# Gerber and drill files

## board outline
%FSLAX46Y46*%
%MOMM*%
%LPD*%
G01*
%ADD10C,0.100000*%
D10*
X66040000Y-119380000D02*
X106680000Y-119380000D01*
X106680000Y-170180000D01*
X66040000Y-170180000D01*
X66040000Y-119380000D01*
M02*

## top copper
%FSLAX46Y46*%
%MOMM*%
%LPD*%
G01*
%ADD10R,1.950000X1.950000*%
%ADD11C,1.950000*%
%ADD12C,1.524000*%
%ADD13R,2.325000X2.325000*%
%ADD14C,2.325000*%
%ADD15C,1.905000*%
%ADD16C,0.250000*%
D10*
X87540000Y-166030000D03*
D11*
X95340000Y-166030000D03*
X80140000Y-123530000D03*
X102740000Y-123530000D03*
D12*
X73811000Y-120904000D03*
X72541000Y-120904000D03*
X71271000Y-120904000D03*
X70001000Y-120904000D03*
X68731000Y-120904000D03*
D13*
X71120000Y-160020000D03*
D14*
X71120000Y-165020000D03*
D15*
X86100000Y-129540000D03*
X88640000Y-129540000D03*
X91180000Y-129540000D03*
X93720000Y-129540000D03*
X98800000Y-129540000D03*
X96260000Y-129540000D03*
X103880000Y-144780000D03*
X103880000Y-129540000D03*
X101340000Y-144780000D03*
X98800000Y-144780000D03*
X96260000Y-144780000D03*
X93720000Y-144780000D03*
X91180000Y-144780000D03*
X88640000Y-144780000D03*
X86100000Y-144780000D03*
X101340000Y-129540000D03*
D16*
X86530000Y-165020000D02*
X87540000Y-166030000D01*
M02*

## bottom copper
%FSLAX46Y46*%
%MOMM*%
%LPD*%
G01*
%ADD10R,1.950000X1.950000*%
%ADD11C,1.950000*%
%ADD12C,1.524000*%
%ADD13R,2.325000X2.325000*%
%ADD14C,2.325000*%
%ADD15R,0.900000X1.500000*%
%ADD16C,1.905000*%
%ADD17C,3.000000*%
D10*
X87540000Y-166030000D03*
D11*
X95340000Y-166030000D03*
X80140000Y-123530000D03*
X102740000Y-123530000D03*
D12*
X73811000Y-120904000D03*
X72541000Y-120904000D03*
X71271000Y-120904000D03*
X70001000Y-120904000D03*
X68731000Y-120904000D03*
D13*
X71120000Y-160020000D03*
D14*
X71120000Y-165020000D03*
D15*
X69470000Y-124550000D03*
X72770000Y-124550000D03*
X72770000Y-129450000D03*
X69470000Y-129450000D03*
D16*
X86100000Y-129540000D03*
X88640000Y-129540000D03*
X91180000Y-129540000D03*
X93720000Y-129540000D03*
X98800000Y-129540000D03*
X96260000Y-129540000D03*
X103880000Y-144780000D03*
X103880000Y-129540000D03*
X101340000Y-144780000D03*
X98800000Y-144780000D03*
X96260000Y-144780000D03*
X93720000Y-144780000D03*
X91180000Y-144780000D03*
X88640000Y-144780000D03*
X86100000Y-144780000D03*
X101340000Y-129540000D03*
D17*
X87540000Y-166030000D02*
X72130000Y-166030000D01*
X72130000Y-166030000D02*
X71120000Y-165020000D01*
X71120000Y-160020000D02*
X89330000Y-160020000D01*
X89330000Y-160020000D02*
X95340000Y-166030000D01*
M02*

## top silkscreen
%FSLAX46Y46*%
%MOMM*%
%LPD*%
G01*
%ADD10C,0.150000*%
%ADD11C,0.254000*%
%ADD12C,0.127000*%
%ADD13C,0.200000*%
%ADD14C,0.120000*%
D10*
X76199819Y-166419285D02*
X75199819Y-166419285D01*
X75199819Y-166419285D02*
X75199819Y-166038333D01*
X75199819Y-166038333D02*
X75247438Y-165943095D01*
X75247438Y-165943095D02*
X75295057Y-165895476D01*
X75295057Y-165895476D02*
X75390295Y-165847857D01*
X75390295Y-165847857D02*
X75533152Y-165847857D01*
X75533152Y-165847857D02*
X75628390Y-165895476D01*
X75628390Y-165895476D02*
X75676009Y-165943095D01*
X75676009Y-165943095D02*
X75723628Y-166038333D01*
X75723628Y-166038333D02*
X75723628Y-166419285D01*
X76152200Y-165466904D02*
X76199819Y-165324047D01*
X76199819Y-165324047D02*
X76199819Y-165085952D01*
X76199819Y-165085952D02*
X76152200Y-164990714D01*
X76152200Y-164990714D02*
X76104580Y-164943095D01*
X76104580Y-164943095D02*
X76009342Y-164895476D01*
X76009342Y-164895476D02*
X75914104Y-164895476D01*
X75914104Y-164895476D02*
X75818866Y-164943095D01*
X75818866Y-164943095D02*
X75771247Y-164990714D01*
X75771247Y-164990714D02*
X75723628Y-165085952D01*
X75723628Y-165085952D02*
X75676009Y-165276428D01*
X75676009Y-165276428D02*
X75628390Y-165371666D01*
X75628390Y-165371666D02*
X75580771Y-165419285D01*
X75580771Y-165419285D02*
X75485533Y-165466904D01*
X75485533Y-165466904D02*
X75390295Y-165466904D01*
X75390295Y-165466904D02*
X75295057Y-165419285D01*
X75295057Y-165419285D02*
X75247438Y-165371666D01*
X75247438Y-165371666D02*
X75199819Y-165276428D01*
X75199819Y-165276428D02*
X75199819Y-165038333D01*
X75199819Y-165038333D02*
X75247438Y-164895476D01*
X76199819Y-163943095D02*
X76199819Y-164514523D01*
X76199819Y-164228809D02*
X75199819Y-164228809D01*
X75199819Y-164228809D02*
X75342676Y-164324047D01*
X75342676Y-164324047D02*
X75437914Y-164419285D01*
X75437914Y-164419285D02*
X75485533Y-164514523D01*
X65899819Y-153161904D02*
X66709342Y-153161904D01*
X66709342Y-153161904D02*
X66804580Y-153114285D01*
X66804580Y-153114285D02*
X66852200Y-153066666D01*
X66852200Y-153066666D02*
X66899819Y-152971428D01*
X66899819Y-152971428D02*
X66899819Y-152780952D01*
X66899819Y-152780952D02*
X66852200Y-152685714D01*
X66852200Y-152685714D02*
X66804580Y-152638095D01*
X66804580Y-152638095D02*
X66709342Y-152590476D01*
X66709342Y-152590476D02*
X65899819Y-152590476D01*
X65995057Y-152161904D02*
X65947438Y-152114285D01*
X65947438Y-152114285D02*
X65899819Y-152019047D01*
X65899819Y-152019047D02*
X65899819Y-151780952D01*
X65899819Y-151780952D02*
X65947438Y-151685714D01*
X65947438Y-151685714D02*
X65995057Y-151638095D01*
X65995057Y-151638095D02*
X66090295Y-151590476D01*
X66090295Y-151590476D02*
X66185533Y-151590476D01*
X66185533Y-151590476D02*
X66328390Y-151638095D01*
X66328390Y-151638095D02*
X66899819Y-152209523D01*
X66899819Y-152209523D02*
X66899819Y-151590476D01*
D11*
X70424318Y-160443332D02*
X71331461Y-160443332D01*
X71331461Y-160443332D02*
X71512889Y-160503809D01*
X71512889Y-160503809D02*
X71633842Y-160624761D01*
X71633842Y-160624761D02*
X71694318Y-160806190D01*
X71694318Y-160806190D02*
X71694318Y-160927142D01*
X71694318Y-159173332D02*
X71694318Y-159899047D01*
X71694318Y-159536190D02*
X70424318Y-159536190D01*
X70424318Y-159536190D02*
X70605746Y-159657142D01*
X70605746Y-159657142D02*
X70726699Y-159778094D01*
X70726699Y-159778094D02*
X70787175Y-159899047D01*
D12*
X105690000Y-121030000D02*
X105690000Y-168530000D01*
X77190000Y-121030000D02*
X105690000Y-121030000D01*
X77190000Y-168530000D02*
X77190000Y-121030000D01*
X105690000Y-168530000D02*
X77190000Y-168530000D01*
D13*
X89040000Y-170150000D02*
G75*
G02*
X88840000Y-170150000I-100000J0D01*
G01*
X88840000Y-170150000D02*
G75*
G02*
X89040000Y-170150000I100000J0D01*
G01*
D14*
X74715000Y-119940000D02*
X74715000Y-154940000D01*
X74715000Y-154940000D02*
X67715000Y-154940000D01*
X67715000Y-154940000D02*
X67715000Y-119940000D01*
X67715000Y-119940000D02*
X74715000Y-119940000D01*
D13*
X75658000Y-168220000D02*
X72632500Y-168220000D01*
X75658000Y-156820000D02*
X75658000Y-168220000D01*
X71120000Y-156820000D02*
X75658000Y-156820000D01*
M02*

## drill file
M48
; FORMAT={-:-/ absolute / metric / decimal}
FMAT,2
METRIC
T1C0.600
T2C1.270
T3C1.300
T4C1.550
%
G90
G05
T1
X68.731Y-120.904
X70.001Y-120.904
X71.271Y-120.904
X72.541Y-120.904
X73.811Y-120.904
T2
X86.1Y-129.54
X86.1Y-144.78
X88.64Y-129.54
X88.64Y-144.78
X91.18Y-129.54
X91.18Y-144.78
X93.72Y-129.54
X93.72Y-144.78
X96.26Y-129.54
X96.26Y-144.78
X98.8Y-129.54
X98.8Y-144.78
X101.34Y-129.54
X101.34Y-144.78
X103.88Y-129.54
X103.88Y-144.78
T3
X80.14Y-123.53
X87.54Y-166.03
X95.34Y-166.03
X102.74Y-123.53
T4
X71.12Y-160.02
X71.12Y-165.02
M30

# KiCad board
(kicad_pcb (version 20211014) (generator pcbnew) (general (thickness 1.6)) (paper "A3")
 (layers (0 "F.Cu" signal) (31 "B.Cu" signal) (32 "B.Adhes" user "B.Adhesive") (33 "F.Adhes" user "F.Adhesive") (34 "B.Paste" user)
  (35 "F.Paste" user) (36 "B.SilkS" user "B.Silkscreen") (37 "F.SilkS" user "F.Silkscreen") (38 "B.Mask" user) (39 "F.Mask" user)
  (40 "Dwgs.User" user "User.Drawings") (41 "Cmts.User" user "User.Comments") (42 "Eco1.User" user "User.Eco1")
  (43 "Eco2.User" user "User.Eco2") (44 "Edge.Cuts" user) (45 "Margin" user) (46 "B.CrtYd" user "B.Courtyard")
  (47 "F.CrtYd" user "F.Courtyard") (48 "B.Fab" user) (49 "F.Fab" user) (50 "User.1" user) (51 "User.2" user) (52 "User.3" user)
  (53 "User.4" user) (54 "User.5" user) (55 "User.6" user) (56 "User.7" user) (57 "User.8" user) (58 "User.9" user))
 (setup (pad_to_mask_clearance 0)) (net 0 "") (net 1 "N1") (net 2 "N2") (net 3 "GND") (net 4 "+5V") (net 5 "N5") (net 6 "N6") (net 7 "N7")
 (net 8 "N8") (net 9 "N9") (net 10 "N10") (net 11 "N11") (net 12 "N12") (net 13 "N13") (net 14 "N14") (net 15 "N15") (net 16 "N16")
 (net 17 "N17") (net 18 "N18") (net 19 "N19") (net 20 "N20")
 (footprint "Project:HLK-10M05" (layer "F.Cu") (at 91.44 144.78 90)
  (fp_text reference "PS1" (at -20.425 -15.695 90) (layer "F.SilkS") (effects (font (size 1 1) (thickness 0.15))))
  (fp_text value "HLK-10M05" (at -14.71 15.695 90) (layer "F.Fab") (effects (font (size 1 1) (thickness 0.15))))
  (fp_line (start 23.75 14.25) (end -23.75 14.25) (layer "F.SilkS") (width 0.127))
  (fp_line (start 23.75 -14.25) (end 23.75 14.25) (layer "F.SilkS") (width 0.127))
  (fp_line (start -23.75 -14.25) (end 23.75 -14.25) (layer "F.SilkS") (width 0.127))
  (fp_line (start -23.75 14.25) (end -23.75 -14.25) (layer "F.SilkS") (width 0.127))
  (fp_circle (center -25.37 -2.5) (end -25.27 -2.5) (layer "F.SilkS") (width 0.2) (fill none))
  (pad "1" thru_hole rect (at -21.25 -3.9 90) (size 1.95 1.95) (drill 1.3) (layers *.Cu *.Mask) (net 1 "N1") (solder_mask_margin 0.102))
  (pad "2" thru_hole circle (at -21.25 3.9 90) (size 1.95 1.95) (drill 1.3) (layers *.Cu *.Mask) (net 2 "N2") (solder_mask_margin 0.102))
  (pad "3" thru_hole circle (at 21.25 -11.3 90) (size 1.95 1.95) (drill 1.3) (layers *.Cu *.Mask) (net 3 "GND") (solder_mask_margin 0.102))
  (pad "4" thru_hole circle (at 21.25 11.3 90) (size 1.95 1.95) (drill 1.3) (layers *.Cu *.Mask) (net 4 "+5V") (solder_mask_margin 0.102)))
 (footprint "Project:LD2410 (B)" (layer "F.Cu") (at 67.715 154.94 90)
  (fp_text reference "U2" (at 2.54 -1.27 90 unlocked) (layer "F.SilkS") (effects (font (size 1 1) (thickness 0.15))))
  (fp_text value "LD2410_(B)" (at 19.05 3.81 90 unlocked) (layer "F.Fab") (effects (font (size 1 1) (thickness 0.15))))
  (fp_line (start 35 7) (end 0 7) (layer "F.SilkS") (width 0.12))
  (fp_line (start 0 7) (end 0 0) (layer "F.SilkS") (width 0.12))
  (fp_line (start 0 0) (end 35 0) (layer "F.SilkS") (width 0.12))
  (fp_line (start 35 0) (end 35 7) (layer "F.SilkS") (width 0.12))
  (pad "1" thru_hole circle (at 34.036 6.096 90) (size 1.524 1.524) (drill 0.6) (layers *.Cu *.Mask) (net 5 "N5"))
  (pad "2" thru_hole circle (at 34.036 4.826 90) (size 1.524 1.524) (drill 0.6) (layers *.Cu *.Mask) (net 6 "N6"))
  (pad "3" thru_hole circle (at 34.036 3.556 90) (size 1.524 1.524) (drill 0.6) (layers *.Cu *.Mask) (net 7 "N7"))
  (pad "4" thru_hole circle (at 34.036 2.286 90) (size 1.524 1.524) (drill 0.6) (layers *.Cu *.Mask) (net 3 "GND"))
  (pad "5" thru_hole circle (at 34.036 1.016 90) (size 1.524 1.524) (drill oval 0.6) (layers *.Cu *.Mask) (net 4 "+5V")))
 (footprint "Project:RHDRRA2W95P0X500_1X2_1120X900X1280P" (layer "F.Cu") (at 71.12 160.02 -90)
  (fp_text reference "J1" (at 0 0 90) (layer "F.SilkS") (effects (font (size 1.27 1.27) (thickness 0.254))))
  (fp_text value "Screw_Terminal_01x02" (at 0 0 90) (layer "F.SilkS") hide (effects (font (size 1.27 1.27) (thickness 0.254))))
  (fp_line (start 8.2 -4.538) (end 8.2 -1.5125) (layer "F.SilkS") (width 0.2))
  (fp_line (start -3.2 -4.538) (end 8.2 -4.538) (layer "F.SilkS") (width 0.2))
  (fp_line (start -3.2 0) (end -3.2 -4.538) (layer "F.SilkS") (width 0.2))
  (pad "1" thru_hole rect locked (at 0 0 270) (size 2.325 2.325) (drill 1.55) (layers *.Cu *.Mask) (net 2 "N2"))
  (pad "2" thru_hole circle locked (at 5 0 270) (size 2.325 2.325) (drill 1.55) (layers *.Cu *.Mask) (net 1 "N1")))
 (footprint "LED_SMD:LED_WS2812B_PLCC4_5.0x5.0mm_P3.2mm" (layer "B.Cu") (at 71.12 127 -90)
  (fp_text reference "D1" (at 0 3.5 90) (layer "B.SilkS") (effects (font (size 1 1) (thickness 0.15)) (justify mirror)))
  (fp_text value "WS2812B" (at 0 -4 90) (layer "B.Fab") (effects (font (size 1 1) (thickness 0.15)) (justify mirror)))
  (pad "1" smd rect (at -2.45 1.65 270) (size 1.5 0.9) (layers "B.Cu" "B.Paste" "B.Mask") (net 3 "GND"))
  (pad "2" smd rect (at -2.45 -1.65 270) (size 1.5 0.9) (layers "B.Cu" "B.Paste" "B.Mask") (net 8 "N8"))
  (pad "3" smd rect (at 2.45 -1.65 270) (size 1.5 0.9) (layers "B.Cu" "B.Paste" "B.Mask") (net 4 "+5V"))
  (pad "4" smd rect (at 2.45 1.65 270) (size 1.5 0.9) (layers "B.Cu" "B.Paste" "B.Mask") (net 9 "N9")))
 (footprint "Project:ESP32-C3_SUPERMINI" (layer "B.Cu") (at 93.98 137.16 90)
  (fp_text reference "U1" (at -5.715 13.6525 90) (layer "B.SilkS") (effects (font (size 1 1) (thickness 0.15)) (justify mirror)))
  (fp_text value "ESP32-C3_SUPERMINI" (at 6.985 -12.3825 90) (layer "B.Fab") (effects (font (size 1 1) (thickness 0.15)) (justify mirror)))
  (pad "0" thru_hole circle (at 7.62 -7.88 90) (size 1.905 1.905) (drill 1.27) (layers *.Cu *.Mask) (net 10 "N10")
   (solder_mask_margin 0.102))
  (pad "1" thru_hole circle (at 7.62 -5.34 90) (size 1.905 1.905) (drill 1.27) (layers *.Cu *.Mask) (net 6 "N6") (solder_mask_margin 0.102))
  (pad "2" thru_hole circle (at 7.62 -2.8 90) (size 1.905 1.905) (drill 1.27) (layers *.Cu *.Mask) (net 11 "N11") (solder_mask_margin 0.102))
  (pad "3" thru_hole circle (at 7.62 -0.26 90) (size 1.905 1.905) (drill 1.27) (layers *.Cu *.Mask) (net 7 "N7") (solder_mask_margin 0.102))
  (pad "3.3" thru_hole circle (at 7.62 4.82 90) (size 1.905 1.905) (drill 1.27) (layers *.Cu *.Mask) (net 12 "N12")
   (solder_mask_margin 0.102))
  (pad "4" thru_hole circle (at 7.62 2.28 90) (size 1.905 1.905) (drill 1.27) (layers *.Cu *.Mask) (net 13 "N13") (solder_mask_margin 0.102))
  (pad "5" thru_hole circle (at -7.62 9.9 90) (size 1.905 1.905) (drill 1.27) (layers *.Cu *.Mask) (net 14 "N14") (solder_mask_margin 0.102))
  (pad "5V" thru_hole circle (at 7.62 9.9 90) (size 1.905 1.905) (drill 1.27) (layers *.Cu *.Mask) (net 4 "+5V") (solder_mask_margin 0.102))
  (pad "6" thru_hole circle (at -7.62 7.36 90) (size 1.905 1.905) (drill 1.27) (layers *.Cu *.Mask) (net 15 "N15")
   (solder_mask_margin 0.102))
  (pad "7" thru_hole circle (at -7.62 4.82 90) (size 1.905 1.905) (drill 1.27) (layers *.Cu *.Mask) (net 9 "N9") (solder_mask_margin 0.102))
  (pad "8" thru_hole circle (at -7.62 2.28 90) (size 1.905 1.905) (drill 1.27) (layers *.Cu *.Mask) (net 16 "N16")
   (solder_mask_margin 0.102))
  (pad "9" thru_hole circle (at -7.62 -0.26 90) (size 1.905 1.905) (drill 1.27) (layers *.Cu *.Mask) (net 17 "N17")
   (solder_mask_margin 0.102))
  (pad "10" thru_hole circle (at -7.62 -2.8 90) (size 1.905 1.905) (drill 1.27) (layers *.Cu *.Mask) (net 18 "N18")
   (solder_mask_margin 0.102))
  (pad "20" thru_hole circle (at -7.62 -5.34 90) (size 1.905 1.905) (drill 1.27) (layers *.Cu *.Mask) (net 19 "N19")
   (solder_mask_margin 0.102))
  (pad "21" thru_hole circle (at -7.62 -7.88 90) (size 1.905 1.905) (drill 1.27) (layers *.Cu *.Mask) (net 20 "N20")
   (solder_mask_margin 0.102))
  (pad "G" thru_hole circle (at 7.62 7.36 90) (size 1.905 1.905) (drill 1.27) (layers *.Cu *.Mask) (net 3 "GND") (solder_mask_margin 0.102)))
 (gr_rect (start 66.04 119.38) (end 106.68 170.18) (layer "Edge.Cuts") (width 0.1) (fill none))
 (segment (start 86.53 165.02) (end 87.54 166.03) (width 0.25) (layer "F.Cu") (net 1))
 (segment (start 87.54 166.03) (end 72.13 166.03) (width 3) (layer "B.Cu") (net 1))
 (segment (start 72.13 166.03) (end 71.12 165.02) (width 3) (layer "B.Cu") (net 1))
 (segment (start 71.12 160.02) (end 89.33 160.02) (width 3) (layer "B.Cu") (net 2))
 (segment (start 89.33 160.02) (end 95.34 166.03) (width 3) (layer "B.Cu") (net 2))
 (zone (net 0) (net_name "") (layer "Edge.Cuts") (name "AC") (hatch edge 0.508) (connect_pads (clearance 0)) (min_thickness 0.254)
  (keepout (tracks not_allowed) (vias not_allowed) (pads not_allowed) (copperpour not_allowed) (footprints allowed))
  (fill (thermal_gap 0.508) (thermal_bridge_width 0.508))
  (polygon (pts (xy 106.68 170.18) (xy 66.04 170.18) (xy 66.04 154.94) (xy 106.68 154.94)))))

